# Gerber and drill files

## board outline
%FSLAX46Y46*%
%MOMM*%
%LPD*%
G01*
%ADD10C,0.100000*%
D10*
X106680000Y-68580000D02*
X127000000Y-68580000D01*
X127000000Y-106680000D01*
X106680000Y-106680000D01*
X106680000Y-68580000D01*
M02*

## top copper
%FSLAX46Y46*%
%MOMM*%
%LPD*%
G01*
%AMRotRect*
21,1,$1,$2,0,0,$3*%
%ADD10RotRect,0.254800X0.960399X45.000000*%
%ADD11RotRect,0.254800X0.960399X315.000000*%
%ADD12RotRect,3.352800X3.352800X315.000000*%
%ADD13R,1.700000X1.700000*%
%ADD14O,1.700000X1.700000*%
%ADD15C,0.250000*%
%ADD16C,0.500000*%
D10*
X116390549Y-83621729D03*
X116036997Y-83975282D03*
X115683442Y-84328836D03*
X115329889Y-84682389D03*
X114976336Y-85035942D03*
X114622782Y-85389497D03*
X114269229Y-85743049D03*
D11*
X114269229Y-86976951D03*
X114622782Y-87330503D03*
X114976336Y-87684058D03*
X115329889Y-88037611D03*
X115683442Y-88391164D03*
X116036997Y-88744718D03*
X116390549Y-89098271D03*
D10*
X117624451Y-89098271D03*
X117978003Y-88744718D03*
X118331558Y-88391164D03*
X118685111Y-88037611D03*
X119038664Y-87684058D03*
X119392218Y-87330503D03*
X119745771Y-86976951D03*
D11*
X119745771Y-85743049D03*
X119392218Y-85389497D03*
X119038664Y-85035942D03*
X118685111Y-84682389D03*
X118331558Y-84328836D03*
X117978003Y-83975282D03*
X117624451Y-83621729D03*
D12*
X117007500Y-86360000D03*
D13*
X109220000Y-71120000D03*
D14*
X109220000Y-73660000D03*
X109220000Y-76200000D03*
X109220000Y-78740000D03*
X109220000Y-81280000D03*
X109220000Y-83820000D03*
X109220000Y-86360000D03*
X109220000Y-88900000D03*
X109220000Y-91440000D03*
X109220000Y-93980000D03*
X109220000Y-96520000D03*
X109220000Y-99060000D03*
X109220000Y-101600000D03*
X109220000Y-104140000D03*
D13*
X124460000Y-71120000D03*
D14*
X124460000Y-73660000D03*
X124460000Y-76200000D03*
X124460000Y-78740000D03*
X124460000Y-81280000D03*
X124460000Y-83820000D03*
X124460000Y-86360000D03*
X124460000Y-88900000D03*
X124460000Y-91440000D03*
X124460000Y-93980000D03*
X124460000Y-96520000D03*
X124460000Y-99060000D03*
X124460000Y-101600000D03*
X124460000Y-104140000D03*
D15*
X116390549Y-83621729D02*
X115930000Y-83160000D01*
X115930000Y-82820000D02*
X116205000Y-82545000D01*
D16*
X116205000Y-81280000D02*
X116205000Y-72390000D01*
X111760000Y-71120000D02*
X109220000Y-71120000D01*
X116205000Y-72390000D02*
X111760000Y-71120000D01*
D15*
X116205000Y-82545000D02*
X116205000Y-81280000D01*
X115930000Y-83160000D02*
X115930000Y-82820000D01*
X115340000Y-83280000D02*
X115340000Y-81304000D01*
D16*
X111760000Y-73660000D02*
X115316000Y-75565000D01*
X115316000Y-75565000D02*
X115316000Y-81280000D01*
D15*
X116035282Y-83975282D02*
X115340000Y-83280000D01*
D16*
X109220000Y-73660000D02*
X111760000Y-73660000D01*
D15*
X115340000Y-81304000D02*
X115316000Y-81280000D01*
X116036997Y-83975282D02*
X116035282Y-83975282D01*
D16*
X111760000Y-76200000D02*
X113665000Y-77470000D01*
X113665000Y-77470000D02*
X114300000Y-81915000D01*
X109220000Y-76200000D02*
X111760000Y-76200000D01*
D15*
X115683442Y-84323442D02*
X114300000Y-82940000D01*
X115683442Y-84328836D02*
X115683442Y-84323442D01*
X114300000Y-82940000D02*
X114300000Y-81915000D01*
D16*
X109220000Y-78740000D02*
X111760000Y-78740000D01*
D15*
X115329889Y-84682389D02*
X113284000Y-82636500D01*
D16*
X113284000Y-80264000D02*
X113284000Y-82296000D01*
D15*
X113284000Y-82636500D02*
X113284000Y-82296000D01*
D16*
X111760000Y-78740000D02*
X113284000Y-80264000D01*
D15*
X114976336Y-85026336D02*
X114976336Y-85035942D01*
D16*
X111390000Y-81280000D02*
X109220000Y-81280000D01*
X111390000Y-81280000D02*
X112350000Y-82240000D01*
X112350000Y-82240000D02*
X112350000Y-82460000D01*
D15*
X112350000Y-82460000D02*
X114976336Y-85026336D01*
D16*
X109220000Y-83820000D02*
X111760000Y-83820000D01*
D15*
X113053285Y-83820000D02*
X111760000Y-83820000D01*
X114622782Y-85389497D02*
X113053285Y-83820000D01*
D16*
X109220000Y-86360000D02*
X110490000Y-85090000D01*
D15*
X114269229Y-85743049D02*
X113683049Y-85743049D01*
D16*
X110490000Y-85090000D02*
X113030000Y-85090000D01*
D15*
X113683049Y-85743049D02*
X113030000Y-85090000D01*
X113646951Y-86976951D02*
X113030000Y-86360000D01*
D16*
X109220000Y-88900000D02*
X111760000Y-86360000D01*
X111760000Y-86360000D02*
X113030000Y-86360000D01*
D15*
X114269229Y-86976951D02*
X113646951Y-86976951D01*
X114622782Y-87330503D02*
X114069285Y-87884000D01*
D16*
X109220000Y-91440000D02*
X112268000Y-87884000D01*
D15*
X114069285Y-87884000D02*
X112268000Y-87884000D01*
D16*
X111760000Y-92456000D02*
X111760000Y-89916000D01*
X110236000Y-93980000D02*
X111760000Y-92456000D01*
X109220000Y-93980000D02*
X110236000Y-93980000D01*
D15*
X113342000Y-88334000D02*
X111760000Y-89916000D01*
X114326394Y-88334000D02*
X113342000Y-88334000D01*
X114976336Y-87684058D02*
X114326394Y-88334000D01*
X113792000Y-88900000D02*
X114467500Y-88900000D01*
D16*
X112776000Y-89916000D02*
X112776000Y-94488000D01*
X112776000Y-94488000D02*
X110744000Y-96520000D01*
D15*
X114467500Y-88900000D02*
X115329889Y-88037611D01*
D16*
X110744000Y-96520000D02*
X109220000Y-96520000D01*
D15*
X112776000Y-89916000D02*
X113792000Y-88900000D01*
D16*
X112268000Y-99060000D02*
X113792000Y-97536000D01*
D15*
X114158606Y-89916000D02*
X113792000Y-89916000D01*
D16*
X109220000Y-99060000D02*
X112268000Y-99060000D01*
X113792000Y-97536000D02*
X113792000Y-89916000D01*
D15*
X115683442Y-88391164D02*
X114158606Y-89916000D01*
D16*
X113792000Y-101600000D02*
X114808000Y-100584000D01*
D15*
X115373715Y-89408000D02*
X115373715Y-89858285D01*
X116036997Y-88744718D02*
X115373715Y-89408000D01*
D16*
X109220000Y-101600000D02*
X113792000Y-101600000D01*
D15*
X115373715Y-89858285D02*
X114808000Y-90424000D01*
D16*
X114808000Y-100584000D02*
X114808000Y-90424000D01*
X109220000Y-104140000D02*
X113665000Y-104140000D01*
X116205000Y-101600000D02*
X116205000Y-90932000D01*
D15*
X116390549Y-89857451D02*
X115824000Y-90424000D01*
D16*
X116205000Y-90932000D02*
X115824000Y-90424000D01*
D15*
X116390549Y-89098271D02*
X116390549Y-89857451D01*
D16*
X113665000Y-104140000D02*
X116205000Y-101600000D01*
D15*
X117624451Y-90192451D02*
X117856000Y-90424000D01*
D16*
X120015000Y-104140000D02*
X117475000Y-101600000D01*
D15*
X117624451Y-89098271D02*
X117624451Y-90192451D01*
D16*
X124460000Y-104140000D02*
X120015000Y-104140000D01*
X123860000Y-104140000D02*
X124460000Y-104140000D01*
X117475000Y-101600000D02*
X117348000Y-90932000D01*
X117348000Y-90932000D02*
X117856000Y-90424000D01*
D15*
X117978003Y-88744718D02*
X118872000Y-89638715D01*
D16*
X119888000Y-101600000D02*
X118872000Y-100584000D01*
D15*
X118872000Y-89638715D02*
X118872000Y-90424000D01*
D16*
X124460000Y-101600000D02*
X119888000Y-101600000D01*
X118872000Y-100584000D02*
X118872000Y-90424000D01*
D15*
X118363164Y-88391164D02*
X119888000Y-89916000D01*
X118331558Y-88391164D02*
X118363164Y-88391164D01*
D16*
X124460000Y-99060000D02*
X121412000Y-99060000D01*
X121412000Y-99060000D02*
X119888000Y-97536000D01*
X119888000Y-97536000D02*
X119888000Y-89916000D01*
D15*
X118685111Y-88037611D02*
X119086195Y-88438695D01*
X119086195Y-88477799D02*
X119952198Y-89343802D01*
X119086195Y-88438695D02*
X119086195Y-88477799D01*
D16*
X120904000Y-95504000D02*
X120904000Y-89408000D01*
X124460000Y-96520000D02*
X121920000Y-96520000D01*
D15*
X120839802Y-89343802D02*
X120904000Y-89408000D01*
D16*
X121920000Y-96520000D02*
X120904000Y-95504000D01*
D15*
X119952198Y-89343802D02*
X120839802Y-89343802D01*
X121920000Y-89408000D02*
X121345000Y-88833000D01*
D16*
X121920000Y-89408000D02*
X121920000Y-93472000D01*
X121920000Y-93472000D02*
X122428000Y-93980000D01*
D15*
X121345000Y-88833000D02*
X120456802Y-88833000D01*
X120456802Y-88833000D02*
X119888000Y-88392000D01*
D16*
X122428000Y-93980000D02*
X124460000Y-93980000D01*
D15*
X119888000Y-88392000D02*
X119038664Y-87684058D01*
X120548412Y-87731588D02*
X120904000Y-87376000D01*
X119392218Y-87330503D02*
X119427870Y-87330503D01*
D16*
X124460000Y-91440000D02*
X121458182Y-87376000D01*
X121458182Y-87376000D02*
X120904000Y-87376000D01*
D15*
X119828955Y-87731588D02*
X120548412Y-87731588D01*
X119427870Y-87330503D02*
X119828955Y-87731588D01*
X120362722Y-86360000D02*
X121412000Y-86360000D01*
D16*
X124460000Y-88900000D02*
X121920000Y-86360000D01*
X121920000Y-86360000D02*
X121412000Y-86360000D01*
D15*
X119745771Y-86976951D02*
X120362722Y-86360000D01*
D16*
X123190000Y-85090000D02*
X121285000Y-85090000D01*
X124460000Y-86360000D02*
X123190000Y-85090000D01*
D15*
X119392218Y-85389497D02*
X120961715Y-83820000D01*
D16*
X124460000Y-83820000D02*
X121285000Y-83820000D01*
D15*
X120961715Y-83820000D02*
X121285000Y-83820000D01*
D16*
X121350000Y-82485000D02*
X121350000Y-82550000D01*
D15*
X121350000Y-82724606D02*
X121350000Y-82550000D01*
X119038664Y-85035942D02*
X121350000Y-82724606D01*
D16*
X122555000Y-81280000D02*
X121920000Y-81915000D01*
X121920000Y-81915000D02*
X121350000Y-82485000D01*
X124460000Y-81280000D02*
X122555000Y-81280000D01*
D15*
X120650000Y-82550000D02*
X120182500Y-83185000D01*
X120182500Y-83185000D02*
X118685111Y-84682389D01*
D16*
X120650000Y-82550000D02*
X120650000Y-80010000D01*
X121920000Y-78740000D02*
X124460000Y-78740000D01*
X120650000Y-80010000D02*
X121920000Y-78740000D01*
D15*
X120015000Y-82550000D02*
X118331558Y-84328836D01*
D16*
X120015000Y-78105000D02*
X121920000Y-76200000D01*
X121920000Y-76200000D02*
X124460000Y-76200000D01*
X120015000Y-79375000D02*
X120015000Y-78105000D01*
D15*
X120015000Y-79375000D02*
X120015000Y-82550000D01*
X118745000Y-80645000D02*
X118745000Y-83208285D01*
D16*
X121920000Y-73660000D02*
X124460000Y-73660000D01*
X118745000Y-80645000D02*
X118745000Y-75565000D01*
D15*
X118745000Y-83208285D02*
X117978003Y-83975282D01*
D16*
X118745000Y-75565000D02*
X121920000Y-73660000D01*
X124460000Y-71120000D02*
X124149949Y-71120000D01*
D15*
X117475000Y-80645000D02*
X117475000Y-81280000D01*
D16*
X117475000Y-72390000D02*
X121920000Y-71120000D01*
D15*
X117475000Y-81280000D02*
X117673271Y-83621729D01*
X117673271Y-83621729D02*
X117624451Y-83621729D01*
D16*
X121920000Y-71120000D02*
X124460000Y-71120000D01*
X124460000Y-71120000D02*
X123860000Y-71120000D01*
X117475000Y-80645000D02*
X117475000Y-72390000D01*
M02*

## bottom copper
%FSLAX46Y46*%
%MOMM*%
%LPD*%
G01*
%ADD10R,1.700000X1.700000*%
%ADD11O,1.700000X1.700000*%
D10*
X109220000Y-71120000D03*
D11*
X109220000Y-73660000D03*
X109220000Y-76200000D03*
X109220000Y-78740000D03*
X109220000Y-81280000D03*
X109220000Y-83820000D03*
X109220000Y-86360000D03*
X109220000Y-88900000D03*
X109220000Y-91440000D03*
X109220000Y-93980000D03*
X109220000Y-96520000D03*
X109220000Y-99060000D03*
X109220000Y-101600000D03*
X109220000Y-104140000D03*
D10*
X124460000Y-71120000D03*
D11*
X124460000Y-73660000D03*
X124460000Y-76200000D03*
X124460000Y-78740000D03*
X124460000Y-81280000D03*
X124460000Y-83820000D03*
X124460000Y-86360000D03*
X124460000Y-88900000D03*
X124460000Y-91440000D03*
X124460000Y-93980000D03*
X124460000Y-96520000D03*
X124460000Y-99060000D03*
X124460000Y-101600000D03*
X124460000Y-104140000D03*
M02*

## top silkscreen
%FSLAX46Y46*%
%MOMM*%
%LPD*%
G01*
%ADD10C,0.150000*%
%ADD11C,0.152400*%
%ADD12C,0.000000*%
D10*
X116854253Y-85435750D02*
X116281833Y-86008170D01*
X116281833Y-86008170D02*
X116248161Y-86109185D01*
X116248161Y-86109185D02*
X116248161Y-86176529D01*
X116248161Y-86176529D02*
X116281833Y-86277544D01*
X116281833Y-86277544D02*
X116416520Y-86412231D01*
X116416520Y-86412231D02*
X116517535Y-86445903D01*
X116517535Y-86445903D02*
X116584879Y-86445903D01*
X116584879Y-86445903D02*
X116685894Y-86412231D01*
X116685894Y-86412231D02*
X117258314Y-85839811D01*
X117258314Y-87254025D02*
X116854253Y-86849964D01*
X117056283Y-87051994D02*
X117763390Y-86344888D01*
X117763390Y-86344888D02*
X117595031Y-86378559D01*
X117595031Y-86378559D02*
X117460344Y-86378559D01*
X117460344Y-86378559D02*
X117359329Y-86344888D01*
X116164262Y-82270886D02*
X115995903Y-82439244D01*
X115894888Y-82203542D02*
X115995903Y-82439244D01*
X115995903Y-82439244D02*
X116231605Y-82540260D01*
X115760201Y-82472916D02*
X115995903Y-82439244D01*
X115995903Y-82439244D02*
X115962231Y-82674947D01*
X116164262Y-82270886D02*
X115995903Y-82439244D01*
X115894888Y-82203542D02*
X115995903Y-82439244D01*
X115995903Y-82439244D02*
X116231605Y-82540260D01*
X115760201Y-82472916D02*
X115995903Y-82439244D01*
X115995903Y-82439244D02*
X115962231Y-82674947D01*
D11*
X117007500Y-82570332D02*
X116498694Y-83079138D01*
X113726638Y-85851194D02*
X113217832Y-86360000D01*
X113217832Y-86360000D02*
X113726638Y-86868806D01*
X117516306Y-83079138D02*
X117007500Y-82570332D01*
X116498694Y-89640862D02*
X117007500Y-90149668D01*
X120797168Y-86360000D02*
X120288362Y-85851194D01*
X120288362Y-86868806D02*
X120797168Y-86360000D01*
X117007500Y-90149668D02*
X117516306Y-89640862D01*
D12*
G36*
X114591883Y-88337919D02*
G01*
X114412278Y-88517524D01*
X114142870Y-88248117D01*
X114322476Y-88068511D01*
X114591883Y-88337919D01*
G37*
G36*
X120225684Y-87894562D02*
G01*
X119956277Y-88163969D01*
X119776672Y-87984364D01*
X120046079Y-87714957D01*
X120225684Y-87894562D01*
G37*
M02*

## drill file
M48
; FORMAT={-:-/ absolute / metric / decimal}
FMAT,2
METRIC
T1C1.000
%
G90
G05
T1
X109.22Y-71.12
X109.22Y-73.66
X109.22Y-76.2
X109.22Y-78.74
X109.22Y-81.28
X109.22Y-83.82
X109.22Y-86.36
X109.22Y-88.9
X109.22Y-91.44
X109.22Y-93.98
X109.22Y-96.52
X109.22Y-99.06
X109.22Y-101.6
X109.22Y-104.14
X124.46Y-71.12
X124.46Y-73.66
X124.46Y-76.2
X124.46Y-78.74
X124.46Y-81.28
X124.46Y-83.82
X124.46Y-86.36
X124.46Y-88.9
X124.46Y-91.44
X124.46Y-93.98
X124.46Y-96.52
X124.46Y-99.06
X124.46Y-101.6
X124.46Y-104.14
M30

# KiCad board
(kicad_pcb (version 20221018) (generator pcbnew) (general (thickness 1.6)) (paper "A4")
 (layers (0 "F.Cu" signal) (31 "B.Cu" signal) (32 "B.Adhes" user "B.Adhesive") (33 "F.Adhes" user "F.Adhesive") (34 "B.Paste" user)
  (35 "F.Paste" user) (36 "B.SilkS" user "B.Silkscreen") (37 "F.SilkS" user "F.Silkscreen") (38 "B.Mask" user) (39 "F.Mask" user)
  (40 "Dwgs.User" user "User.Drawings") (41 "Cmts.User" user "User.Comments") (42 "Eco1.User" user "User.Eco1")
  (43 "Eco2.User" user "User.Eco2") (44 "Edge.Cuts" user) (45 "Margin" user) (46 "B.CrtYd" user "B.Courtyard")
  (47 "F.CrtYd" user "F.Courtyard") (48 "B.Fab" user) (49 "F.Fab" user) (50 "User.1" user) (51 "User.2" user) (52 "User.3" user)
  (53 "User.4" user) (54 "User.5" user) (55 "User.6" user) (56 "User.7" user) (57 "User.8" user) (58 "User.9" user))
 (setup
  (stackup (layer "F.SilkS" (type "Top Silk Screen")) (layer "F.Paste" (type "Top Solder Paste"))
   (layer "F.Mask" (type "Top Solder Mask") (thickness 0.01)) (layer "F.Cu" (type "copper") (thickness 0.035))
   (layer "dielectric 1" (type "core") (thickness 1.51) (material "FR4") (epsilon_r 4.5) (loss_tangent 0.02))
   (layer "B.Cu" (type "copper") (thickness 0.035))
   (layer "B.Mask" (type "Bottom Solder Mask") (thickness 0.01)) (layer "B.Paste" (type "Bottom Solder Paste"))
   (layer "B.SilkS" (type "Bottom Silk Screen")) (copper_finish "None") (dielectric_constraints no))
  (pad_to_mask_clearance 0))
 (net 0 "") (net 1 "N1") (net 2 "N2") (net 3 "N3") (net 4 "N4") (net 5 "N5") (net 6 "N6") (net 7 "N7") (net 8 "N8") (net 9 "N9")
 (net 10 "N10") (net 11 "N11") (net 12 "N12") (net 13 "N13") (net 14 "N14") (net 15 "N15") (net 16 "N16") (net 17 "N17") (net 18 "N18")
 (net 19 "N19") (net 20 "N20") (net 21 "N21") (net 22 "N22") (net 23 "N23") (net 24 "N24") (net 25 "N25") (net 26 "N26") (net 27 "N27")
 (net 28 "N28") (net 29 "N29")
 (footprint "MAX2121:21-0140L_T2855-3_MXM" (layer "F.Cu") (at 117.0075 86.36 -45)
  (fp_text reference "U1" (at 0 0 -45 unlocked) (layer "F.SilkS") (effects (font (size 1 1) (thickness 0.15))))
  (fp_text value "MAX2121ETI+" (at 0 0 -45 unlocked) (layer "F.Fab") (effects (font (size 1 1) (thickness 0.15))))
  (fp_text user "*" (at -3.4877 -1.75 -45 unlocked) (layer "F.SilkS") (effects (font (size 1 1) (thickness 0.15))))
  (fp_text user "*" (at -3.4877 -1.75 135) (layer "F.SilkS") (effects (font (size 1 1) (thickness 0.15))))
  (fp_line (start -2.6797 -2.6797) (end -2.6797 -1.96014) (stroke (width 0.1524) (type solid)) (layer "F.SilkS"))
  (fp_line (start -2.6797 1.96014) (end -2.6797 2.6797) (stroke (width 0.1524) (type solid)) (layer "F.SilkS"))
  (fp_line (start -2.6797 2.6797) (end -1.96014 2.6797) (stroke (width 0.1524) (type solid)) (layer "F.SilkS"))
  (fp_line (start -1.96014 -2.6797) (end -2.6797 -2.6797) (stroke (width 0.1524) (type solid)) (layer "F.SilkS"))
  (fp_line (start 1.96014 2.6797) (end 2.6797 2.6797) (stroke (width 0.1524) (type solid)) (layer "F.SilkS"))
  (fp_line (start 2.6797 -2.6797) (end 1.96014 -2.6797) (stroke (width 0.1524) (type solid)) (layer "F.SilkS"))
  (fp_line (start 2.6797 -1.96014) (end 2.6797 -2.6797) (stroke (width 0.1524) (type solid)) (layer "F.SilkS"))
  (fp_line (start 2.6797 2.6797) (end 2.6797 1.96014) (stroke (width 0.1524) (type solid)) (layer "F.SilkS"))
  (fp_poly
   (pts (xy -0.690499 3.106699) (xy -0.690499 3.360699) (xy -0.309499 3.360699) (xy -0.309499 3.106699)) (stroke (width 0) (type solid))
   (fill solid) (layer "F.SilkS"))
  (fp_poly
   (pts (xy 3.360699 -1.190501) (xy 3.360699 -0.809501) (xy 3.106699 -0.809501) (xy 3.106699 -1.190501)) (stroke (width 0) (type solid))
   (fill solid) (layer "F.SilkS"))
  (pad "1" smd rect (at -2.3725 -1.5 45) (size 0.2548 0.960399) (layers "F.Cu" "F.Paste" "F.Mask") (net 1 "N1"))
  (pad "2" smd rect (at -2.3725 -1.000001 45) (size 0.2548 0.960399) (layers "F.Cu" "F.Paste" "F.Mask") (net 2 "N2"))
  (pad "3" smd rect (at -2.3725 -0.499999 45) (size 0.2548 0.960399) (layers "F.Cu" "F.Paste" "F.Mask") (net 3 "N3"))
  (pad "4" smd rect (at -2.3725 0 45) (size 0.2548 0.960399) (layers "F.Cu" "F.Paste" "F.Mask") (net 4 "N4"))
  (pad "5" smd rect (at -2.3725 0.499999 45) (size 0.2548 0.960399) (layers "F.Cu" "F.Paste" "F.Mask") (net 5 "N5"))
  (pad "6" smd rect (at -2.3725 1.000001 45) (size 0.2548 0.960399) (layers "F.Cu" "F.Paste" "F.Mask") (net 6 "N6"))
  (pad "7" smd rect (at -2.3725 1.5 45) (size 0.2548 0.960399) (layers "F.Cu" "F.Paste" "F.Mask") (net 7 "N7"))
  (pad "8" smd rect (at -1.5 2.3725 315) (size 0.2548 0.960399) (layers "F.Cu" "F.Paste" "F.Mask") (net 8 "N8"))
  (pad "9" smd rect (at -1.000001 2.3725 315) (size 0.2548 0.960399) (layers "F.Cu" "F.Paste" "F.Mask") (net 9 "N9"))
  (pad "10" smd rect (at -0.499999 2.3725 315) (size 0.2548 0.960399) (layers "F.Cu" "F.Paste" "F.Mask") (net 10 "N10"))
  (pad "11" smd rect (at 0 2.3725 315) (size 0.2548 0.960399) (layers "F.Cu" "F.Paste" "F.Mask") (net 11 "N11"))
  (pad "12" smd rect (at 0.499999 2.3725 315) (size 0.2548 0.960399) (layers "F.Cu" "F.Paste" "F.Mask") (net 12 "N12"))
  (pad "13" smd rect (at 1.000001 2.3725 315) (size 0.2548 0.960399) (layers "F.Cu" "F.Paste" "F.Mask") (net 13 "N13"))
  (pad "14" smd rect (at 1.5 2.3725 315) (size 0.2548 0.960399) (layers "F.Cu" "F.Paste" "F.Mask") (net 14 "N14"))
  (pad "15" smd rect (at 2.3725 1.5 45) (size 0.2548 0.960399) (layers "F.Cu" "F.Paste" "F.Mask") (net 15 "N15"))
  (pad "16" smd rect (at 2.3725 1.000001 45) (size 0.2548 0.960399) (layers "F.Cu" "F.Paste" "F.Mask") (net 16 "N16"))
  (pad "17" smd rect (at 2.3725 0.499999 45) (size 0.2548 0.960399) (layers "F.Cu" "F.Paste" "F.Mask") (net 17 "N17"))
  (pad "18" smd rect (at 2.3725 0 45) (size 0.2548 0.960399) (layers "F.Cu" "F.Paste" "F.Mask") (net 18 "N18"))
  (pad "19" smd rect (at 2.3725 -0.499999 45) (size 0.2548 0.960399) (layers "F.Cu" "F.Paste" "F.Mask") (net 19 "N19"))
  (pad "20" smd rect (at 2.3725 -1.000001 45) (size 0.2548 0.960399) (layers "F.Cu" "F.Paste" "F.Mask") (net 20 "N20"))
  (pad "21" smd rect (at 2.3725 -1.5 45) (size 0.2548 0.960399) (layers "F.Cu" "F.Paste" "F.Mask") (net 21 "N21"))
  (pad "22" smd rect (at 1.5 -2.3725 315) (size 0.2548 0.960399) (layers "F.Cu" "F.Paste" "F.Mask") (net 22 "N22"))
  (pad "23" smd rect (at 1.000001 -2.3725 315) (size 0.2548 0.960399) (layers "F.Cu" "F.Paste" "F.Mask") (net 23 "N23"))
  (pad "24" smd rect (at 0.499999 -2.3725 315) (size 0.2548 0.960399) (layers "F.Cu" "F.Paste" "F.Mask") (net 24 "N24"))
  (pad "25" smd rect (at 0 -2.3725 315) (size 0.2548 0.960399) (layers "F.Cu" "F.Paste" "F.Mask") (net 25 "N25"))
  (pad "26" smd rect (at -0.499999 -2.3725 315) (size 0.2548 0.960399) (layers "F.Cu" "F.Paste" "F.Mask") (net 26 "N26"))
  (pad "27" smd rect (at -1.000001 -2.3725 315) (size 0.2548 0.960399) (layers "F.Cu" "F.Paste" "F.Mask") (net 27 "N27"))
  (pad "28" smd rect (at -1.5 -2.3725 315) (size 0.2548 0.960399) (layers "F.Cu" "F.Paste" "F.Mask") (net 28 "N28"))
  (pad "29" smd rect (at 0 0 315) (size 3.3528 3.3528) (layers "F.Cu" "F.Mask") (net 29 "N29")))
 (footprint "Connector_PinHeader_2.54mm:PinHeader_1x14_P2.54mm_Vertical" (layer "B.Cu") (at 109.22 71.12 180)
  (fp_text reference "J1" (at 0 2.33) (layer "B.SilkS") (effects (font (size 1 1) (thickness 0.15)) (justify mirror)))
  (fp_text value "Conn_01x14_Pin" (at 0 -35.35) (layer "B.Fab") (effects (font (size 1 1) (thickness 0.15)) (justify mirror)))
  (pad "1" thru_hole rect (at 0 0 180) (size 1.7 1.7) (drill 1) (layers "*.Cu" "*.Mask") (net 1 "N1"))
  (pad "2" thru_hole oval (at 0 -2.54 180) (size 1.7 1.7) (drill 1) (layers "*.Cu" "*.Mask") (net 2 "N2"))
  (pad "3" thru_hole oval (at 0 -5.08 180) (size 1.7 1.7) (drill 1) (layers "*.Cu" "*.Mask") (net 3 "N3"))
  (pad "4" thru_hole oval (at 0 -7.62 180) (size 1.7 1.7) (drill 1) (layers "*.Cu" "*.Mask") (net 4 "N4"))
  (pad "5" thru_hole oval (at 0 -10.16 180) (size 1.7 1.7) (drill 1) (layers "*.Cu" "*.Mask") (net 5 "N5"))
  (pad "6" thru_hole oval (at 0 -12.7 180) (size 1.7 1.7) (drill 1) (layers "*.Cu" "*.Mask") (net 6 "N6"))
  (pad "7" thru_hole oval (at 0 -15.24 180) (size 1.7 1.7) (drill 1) (layers "*.Cu" "*.Mask") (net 7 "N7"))
  (pad "8" thru_hole oval (at 0 -17.78 180) (size 1.7 1.7) (drill 1) (layers "*.Cu" "*.Mask") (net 8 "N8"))
  (pad "9" thru_hole oval (at 0 -20.32 180) (size 1.7 1.7) (drill 1) (layers "*.Cu" "*.Mask") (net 9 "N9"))
  (pad "10" thru_hole oval (at 0 -22.86 180) (size 1.7 1.7) (drill 1) (layers "*.Cu" "*.Mask") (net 10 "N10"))
  (pad "11" thru_hole oval (at 0 -25.4 180) (size 1.7 1.7) (drill 1) (layers "*.Cu" "*.Mask") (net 11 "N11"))
  (pad "12" thru_hole oval (at 0 -27.94 180) (size 1.7 1.7) (drill 1) (layers "*.Cu" "*.Mask") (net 12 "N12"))
  (pad "13" thru_hole oval (at 0 -30.48 180) (size 1.7 1.7) (drill 1) (layers "*.Cu" "*.Mask") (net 13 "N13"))
  (pad "14" thru_hole oval (at 0 -33.02 180) (size 1.7 1.7) (drill 1) (layers "*.Cu" "*.Mask") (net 14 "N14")))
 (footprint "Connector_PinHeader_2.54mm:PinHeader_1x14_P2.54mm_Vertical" (layer "B.Cu") (at 124.46 71.12 180)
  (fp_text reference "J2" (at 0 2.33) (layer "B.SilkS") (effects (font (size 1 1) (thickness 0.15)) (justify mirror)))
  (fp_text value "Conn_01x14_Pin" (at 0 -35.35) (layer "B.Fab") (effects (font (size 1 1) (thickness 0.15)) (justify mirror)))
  (pad "1" thru_hole rect (at 0 0 180) (size 1.7 1.7) (drill 1) (layers "*.Cu" "*.Mask") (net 28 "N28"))
  (pad "2" thru_hole oval (at 0 -2.54 180) (size 1.7 1.7) (drill 1) (layers "*.Cu" "*.Mask") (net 27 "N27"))
  (pad "3" thru_hole oval (at 0 -5.08 180) (size 1.7 1.7) (drill 1) (layers "*.Cu" "*.Mask") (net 26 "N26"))
  (pad "4" thru_hole oval (at 0 -7.62 180) (size 1.7 1.7) (drill 1) (layers "*.Cu" "*.Mask") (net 25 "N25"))
  (pad "5" thru_hole oval (at 0 -10.16 180) (size 1.7 1.7) (drill 1) (layers "*.Cu" "*.Mask") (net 24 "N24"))
  (pad "6" thru_hole oval (at 0 -12.7 180) (size 1.7 1.7) (drill 1) (layers "*.Cu" "*.Mask") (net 23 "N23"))
  (pad "7" thru_hole oval (at 0 -15.24 180) (size 1.7 1.7) (drill 1) (layers "*.Cu" "*.Mask") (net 22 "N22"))
  (pad "8" thru_hole oval (at 0 -17.78 180) (size 1.7 1.7) (drill 1) (layers "*.Cu" "*.Mask") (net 21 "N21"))
  (pad "9" thru_hole oval (at 0 -20.32 180) (size 1.7 1.7) (drill 1) (layers "*.Cu" "*.Mask") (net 20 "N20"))
  (pad "10" thru_hole oval (at 0 -22.86 180) (size 1.7 1.7) (drill 1) (layers "*.Cu" "*.Mask") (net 19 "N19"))
  (pad "11" thru_hole oval (at 0 -25.4 180) (size 1.7 1.7) (drill 1) (layers "*.Cu" "*.Mask") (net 18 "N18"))
  (pad "12" thru_hole oval (at 0 -27.94 180) (size 1.7 1.7) (drill 1) (layers "*.Cu" "*.Mask") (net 17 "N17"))
  (pad "13" thru_hole oval (at 0 -30.48 180) (size 1.7 1.7) (drill 1) (layers "*.Cu" "*.Mask") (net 16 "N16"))
  (pad "14" thru_hole oval (at 0 -33.02 180) (size 1.7 1.7) (drill 1) (layers "*.Cu" "*.Mask") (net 15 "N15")))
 (gr_rect (start 106.68 68.58) (end 127 106.68) (stroke (width 0.1) (type default)) (fill none) (layer "Edge.Cuts"))
 (segment (start 116.390549 83.621729) (end 115.93 83.16) (width 0.25) (layer "F.Cu") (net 1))
 (segment (start 115.93 82.82) (end 116.205 82.545) (width 0.25) (layer "F.Cu") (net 1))
 (segment (start 116.205 81.28) (end 116.205 72.39) (width 0.5) (layer "F.Cu") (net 1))
 (segment (start 111.76 71.12) (end 109.22 71.12) (width 0.5) (layer "F.Cu") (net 1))
 (segment (start 116.205 72.39) (end 111.76 71.12) (width 0.5) (layer "F.Cu") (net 1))
 (segment (start 116.205 82.545) (end 116.205 81.28) (width 0.25) (layer "F.Cu") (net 1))
 (segment (start 115.93 83.16) (end 115.93 82.82) (width 0.25) (layer "F.Cu") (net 1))
 (segment (start 115.34 83.28) (end 115.34 81.304) (width 0.25) (layer "F.Cu") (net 2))
 (segment (start 111.76 73.66) (end 115.316 75.565) (width 0.5) (layer "F.Cu") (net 2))
 (segment (start 115.316 75.565) (end 115.316 81.28) (width 0.5) (layer "F.Cu") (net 2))
 (segment (start 116.035282 83.975282) (end 115.34 83.28) (width 0.25) (layer "F.Cu") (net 2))
 (segment (start 109.22 73.66) (end 111.76 73.66) (width 0.5) (layer "F.Cu") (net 2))
 (segment (start 115.34 81.304) (end 115.316 81.28) (width 0.25) (layer "F.Cu") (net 2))
 (segment (start 116.036997 83.975282) (end 116.035282 83.975282) (width 0.25) (layer "F.Cu") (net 2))
 (segment (start 111.76 76.2) (end 113.665 77.47) (width 0.5) (layer "F.Cu") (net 3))
 (segment (start 113.665 77.47) (end 114.3 81.915) (width 0.5) (layer "F.Cu") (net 3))
 (segment (start 109.22 76.2) (end 111.76 76.2) (width 0.5) (layer "F.Cu") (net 3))
 (segment (start 115.683442 84.323442) (end 114.3 82.94) (width 0.25) (layer "F.Cu") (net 3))
 (segment (start 115.683442 84.328836) (end 115.683442 84.323442) (width 0.25) (layer "F.Cu") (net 3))
 (segment (start 114.3 82.94) (end 114.3 81.915) (width 0.25) (layer "F.Cu") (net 3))
 (segment (start 109.22 78.74) (end 111.76 78.74) (width 0.5) (layer "F.Cu") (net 4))
 (segment (start 115.329889 84.682389) (end 113.284 82.6365) (width 0.25) (layer "F.Cu") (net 4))
 (segment (start 113.284 80.264) (end 113.284 82.296) (width 0.5) (layer "F.Cu") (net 4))
 (segment (start 113.284 82.6365) (end 113.284 82.296) (width 0.25) (layer "F.Cu") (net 4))
 (segment (start 111.76 78.74) (end 113.284 80.264) (width 0.5) (layer "F.Cu") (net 4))
 (segment (start 114.976336 85.026336) (end 114.976336 85.035942) (width 0.25) (layer "F.Cu") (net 5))
 (segment (start 111.39 81.28) (end 109.22 81.28) (width 0.5) (layer "F.Cu") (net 5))
 (segment (start 111.39 81.28) (end 112.35 82.24) (width 0.5) (layer "F.Cu") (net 5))
 (segment (start 112.35 82.24) (end 112.35 82.46) (width 0.5) (layer "F.Cu") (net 5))
 (segment (start 112.35 82.46) (end 114.976336 85.026336) (width 0.25) (layer "F.Cu") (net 5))
 (segment (start 109.22 83.82) (end 111.76 83.82) (width 0.5) (layer "F.Cu") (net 6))
 (segment (start 113.053285 83.82) (end 111.76 83.82) (width 0.25) (layer "F.Cu") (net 6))
 (segment (start 114.622782 85.389497) (end 113.053285 83.82) (width 0.25) (layer "F.Cu") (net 6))
 (segment (start 109.22 86.36) (end 110.49 85.09) (width 0.5) (layer "F.Cu") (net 7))
 (segment (start 114.269229 85.743049) (end 113.683049 85.743049) (width 0.25) (layer "F.Cu") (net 7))
 (segment (start 110.49 85.09) (end 113.03 85.09) (width 0.5) (layer "F.Cu") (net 7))
 (segment (start 113.683049 85.743049) (end 113.03 85.09) (width 0.25) (layer "F.Cu") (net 7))
 (segment (start 113.646951 86.976951) (end 113.03 86.36) (width 0.25) (layer "F.Cu") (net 8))
 (segment (start 109.22 88.9) (end 111.76 86.36) (width 0.5) (layer "F.Cu") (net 8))
 (segment (start 111.76 86.36) (end 113.03 86.36) (width 0.5) (layer "F.Cu") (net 8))
 (segment (start 114.269229 86.976951) (end 113.646951 86.976951) (width 0.25) (layer "F.Cu") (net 8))
 (segment (start 114.622782 87.330503) (end 114.069285 87.884) (width 0.25) (layer "F.Cu") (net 9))
 (segment (start 109.22 91.44) (end 112.268 87.884) (width 0.5) (layer "F.Cu") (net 9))
 (segment (start 114.069285 87.884) (end 112.268 87.884) (width 0.25) (layer "F.Cu") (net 9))
 (segment (start 111.76 92.456) (end 111.76 89.916) (width 0.5) (layer "F.Cu") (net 10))
 (segment (start 110.236 93.98) (end 111.76 92.456) (width 0.5) (layer "F.Cu") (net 10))
 (segment (start 109.22 93.98) (end 110.236 93.98) (width 0.5) (layer "F.Cu") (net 10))
 (segment (start 113.342 88.334) (end 111.76 89.916) (width 0.25) (layer "F.Cu") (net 10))
 (segment (start 114.326394 88.334) (end 113.342 88.334) (width 0.25) (layer "F.Cu") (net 10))
 (segment (start 114.976336 87.684058) (end 114.326394 88.334) (width 0.25) (layer "F.Cu") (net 10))
 (segment (start 113.792 88.9) (end 114.4675 88.9) (width 0.25) (layer "F.Cu") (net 11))
 (segment (start 112.776 89.916) (end 112.776 94.488) (width 0.5) (layer "F.Cu") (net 11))
 (segment (start 112.776 94.488) (end 110.744 96.52) (width 0.5) (layer "F.Cu") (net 11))
 (segment (start 114.4675 88.9) (end 115.329889 88.037611) (width 0.25) (layer "F.Cu") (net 11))
 (segment (start 110.744 96.52) (end 109.22 96.52) (width 0.5) (layer "F.Cu") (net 11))
 (segment (start 112.776 89.916) (end 113.792 88.9) (width 0.25) (layer "F.Cu") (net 11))
 (segment (start 112.268 99.06) (end 113.792 97.536) (width 0.5) (layer "F.Cu") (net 12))
 (segment (start 114.158606 89.916) (end 113.792 89.916) (width 0.25) (layer "F.Cu") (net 12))
 (segment (start 109.22 99.06) (end 112.268 99.06) (width 0.5) (layer "F.Cu") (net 12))
 (segment (start 113.792 97.536) (end 113.792 89.916) (width 0.5) (layer "F.Cu") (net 12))
 (segment (start 115.683442 88.391164) (end 114.158606 89.916) (width 0.25) (layer "F.Cu") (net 12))
 (segment (start 113.792 101.6) (end 114.808 100.584) (width 0.5) (layer "F.Cu") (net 13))
 (segment (start 115.373715 89.408) (end 115.373715 89.858285) (width 0.25) (layer "F.Cu") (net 13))
 (segment (start 116.036997 88.744718) (end 115.373715 89.408) (width 0.25) (layer "F.Cu") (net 13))
 (segment (start 109.22 101.6) (end 113.792 101.6) (width 0.5) (layer "F.Cu") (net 13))
 (segment (start 115.373715 89.858285) (end 114.808 90.424) (width 0.25) (layer "F.Cu") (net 13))
 (segment (start 114.808 100.584) (end 114.808 90.424) (width 0.5) (layer "F.Cu") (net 13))
 (segment (start 109.22 104.14) (end 113.665 104.14) (width 0.5) (layer "F.Cu") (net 14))
 (segment (start 116.205 101.6) (end 116.205 90.932) (width 0.5) (layer "F.Cu") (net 14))
 (segment (start 116.390549 89.857451) (end 115.824 90.424) (width 0.25) (layer "F.Cu") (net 14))
 (segment (start 116.205 90.932) (end 115.824 90.424) (width 0.5) (layer "F.Cu") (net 14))
 (segment (start 116.390549 89.098271) (end 116.390549 89.857451) (width 0.25) (layer "F.Cu") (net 14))
 (segment (start 113.665 104.14) (end 116.205 101.6) (width 0.5) (layer "F.Cu") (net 14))
 (segment (start 117.624451 90.192451) (end 117.856 90.424) (width 0.25) (layer "F.Cu") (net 15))
 (segment (start 120.015 104.14) (end 117.475 101.6) (width 0.5) (layer "F.Cu") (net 15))
 (segment (start 117.624451 89.098271) (end 117.624451 90.192451) (width 0.25) (layer "F.Cu") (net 15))
 (segment (start 124.46 104.14) (end 120.015 104.14) (width 0.5) (layer "F.Cu") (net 15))
 (segment (start 123.86 104.14) (end 124.46 104.14) (width 0.5) (layer "F.Cu") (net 15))
 (segment (start 117.475 101.6) (end 117.348 90.932) (width 0.5) (layer "F.Cu") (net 15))
 (segment (start 117.348 90.932) (end 117.856 90.424) (width 0.5) (layer "F.Cu") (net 15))
 (segment (start 117.978003 88.744718) (end 118.872 89.638715) (width 0.25) (layer "F.Cu") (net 16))
 (segment (start 119.888 101.6) (end 118.872 100.584) (width 0.5) (layer "F.Cu") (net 16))
 (segment (start 118.872 89.638715) (end 118.872 90.424) (width 0.25) (layer "F.Cu") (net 16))
 (segment (start 124.46 101.6) (end 119.888 101.6) (width 0.5) (layer "F.Cu") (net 16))
 (segment (start 118.872 100.584) (end 118.872 90.424) (width 0.5) (layer "F.Cu") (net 16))
 (segment (start 118.363164 88.391164) (end 119.888 89.916) (width 0.25) (layer "F.Cu") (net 17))
 (segment (start 118.331558 88.391164) (end 118.363164 88.391164) (width 0.25) (layer "F.Cu") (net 17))
 (segment (start 124.46 99.06) (end 121.412 99.06) (width 0.5) (layer "F.Cu") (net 17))
 (segment (start 121.412 99.06) (end 119.888 97.536) (width 0.5) (layer "F.Cu") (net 17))
 (segment (start 119.888 97.536) (end 119.888 89.916) (width 0.5) (layer "F.Cu") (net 17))
 (segment (start 118.685111 88.037611) (end 119.086195 88.438695) (width 0.25) (layer "F.Cu") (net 18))
 (segment (start 119.086195 88.477799) (end 119.952198 89.343802) (width 0.25) (layer "F.Cu") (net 18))
 (segment (start 119.086195 88.438695) (end 119.086195 88.477799) (width 0.25) (layer "F.Cu") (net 18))
 (segment (start 120.904 95.504) (end 120.904 89.408) (width 0.5) (layer "F.Cu") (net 18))
 (segment (start 124.46 96.52) (end 121.92 96.52) (width 0.5) (layer "F.Cu") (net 18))
 (segment (start 120.839802 89.343802) (end 120.904 89.408) (width 0.25) (layer "F.Cu") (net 18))
 (segment (start 121.92 96.52) (end 120.904 95.504) (width 0.5) (layer "F.Cu") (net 18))
 (segment (start 119.952198 89.343802) (end 120.839802 89.343802) (width 0.25) (layer "F.Cu") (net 18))
 (segment (start 121.92 89.408) (end 121.345 88.833) (width 0.25) (layer "F.Cu") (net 19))
 (segment (start 121.92 89.408) (end 121.92 93.472) (width 0.5) (layer "F.Cu") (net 19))
 (segment (start 121.92 93.472) (end 122.428 93.98) (width 0.5) (layer "F.Cu") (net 19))
 (segment (start 121.345 88.833) (end 120.456802 88.833) (width 0.25) (layer "F.Cu") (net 19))
 (segment (start 120.456802 88.833) (end 119.888 88.392) (width 0.25) (layer "F.Cu") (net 19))
 (segment (start 122.428 93.98) (end 124.46 93.98) (width 0.5) (layer "F.Cu") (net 19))
 (segment (start 119.888 88.392) (end 119.038664 87.684058) (width 0.25) (layer "F.Cu") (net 19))
 (segment (start 120.548412 87.731588) (end 120.904 87.376) (width 0.25) (layer "F.Cu") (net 20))
 (segment (start 119.392218 87.330503) (end 119.42787 87.330503) (width 0.25) (layer "F.Cu") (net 20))
 (segment (start 124.46 91.44) (end 121.458182 87.376) (width 0.5) (layer "F.Cu") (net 20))
 (segment (start 121.458182 87.376) (end 120.904 87.376) (width 0.5) (layer "F.Cu") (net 20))
 (segment (start 119.828955 87.731588) (end 120.548412 87.731588) (width 0.25) (layer "F.Cu") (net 20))
 (segment (start 119.42787 87.330503) (end 119.828955 87.731588) (width 0.25) (layer "F.Cu") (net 20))
 (segment (start 120.362722 86.36) (end 121.412 86.36) (width 0.25) (layer "F.Cu") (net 21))
 (segment (start 124.46 88.9) (end 121.92 86.36) (width 0.5) (layer "F.Cu") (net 21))
 (segment (start 121.92 86.36) (end 121.412 86.36) (width 0.5) (layer "F.Cu") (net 21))
 (segment (start 119.745771 86.976951) (end 120.362722 86.36) (width 0.25) (layer "F.Cu") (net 21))
 (segment (start 123.19 85.09) (end 121.285 85.09) (width 0.5) (layer "F.Cu") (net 22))
 (segment (start 124.46 86.36) (end 123.19 85.09) (width 0.5) (layer "F.Cu") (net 22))
 (segment (start 119.392218 85.389497) (end 120.961715 83.82) (width 0.25) (layer "F.Cu") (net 23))
 (segment (start 124.46 83.82) (end 121.285 83.82) (width 0.5) (layer "F.Cu") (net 23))
 (segment (start 120.961715 83.82) (end 121.285 83.82) (width 0.25) (layer "F.Cu") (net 23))
 (segment (start 121.35 82.485) (end 121.35 82.55) (width 0.5) (layer "F.Cu") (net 24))
 (segment (start 121.35 82.724606) (end 121.35 82.55) (width 0.25) (layer "F.Cu") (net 24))
 (segment (start 119.038664 85.035942) (end 121.35 82.724606) (width 0.25) (layer "F.Cu") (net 24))
 (segment (start 122.555 81.28) (end 121.92 81.915) (width 0.5) (layer "F.Cu") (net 24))
 (segment (start 121.92 81.915) (end 121.35 82.485) (width 0.5) (layer "F.Cu") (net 24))
 (segment (start 124.46 81.28) (end 122.555 81.28) (width 0.5) (layer "F.Cu") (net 24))
 (segment (start 120.65 82.55) (end 120.1825 83.185) (width 0.25) (layer "F.Cu") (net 25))
 (segment (start 120.1825 83.185) (end 118.685111 84.682389) (width 0.25) (layer "F.Cu") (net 25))
 (segment (start 120.65 82.55) (end 120.65 80.01) (width 0.5) (layer "F.Cu") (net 25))
 (segment (start 121.92 78.74) (end 124.46 78.74) (width 0.5) (layer "F.Cu") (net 25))
 (segment (start 120.65 80.01) (end 121.92 78.74) (width 0.5) (layer "F.Cu") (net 25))
 (segment (start 120.015 82.55) (end 118.331558 84.328836) (width 0.25) (layer "F.Cu") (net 26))
 (segment (start 120.015 78.105) (end 121.92 76.2) (width 0.5) (layer "F.Cu") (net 26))
 (segment (start 121.92 76.2) (end 124.46 76.2) (width 0.5) (layer "F.Cu") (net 26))
 (segment (start 120.015 79.375) (end 120.015 78.105) (width 0.5) (layer "F.Cu") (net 26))
 (segment (start 120.015 79.375) (end 120.015 82.55) (width 0.25) (layer "F.Cu") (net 26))
 (segment (start 118.745 80.645) (end 118.745 83.208285) (width 0.25) (layer "F.Cu") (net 27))
 (segment (start 121.92 73.66) (end 124.46 73.66) (width 0.5) (layer "F.Cu") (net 27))
 (segment (start 118.745 80.645) (end 118.745 75.565) (width 0.5) (layer "F.Cu") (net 27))
 (segment (start 118.745 83.208285) (end 117.978003 83.975282) (width 0.25) (layer "F.Cu") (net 27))
 (segment (start 118.745 75.565) (end 121.92 73.66) (width 0.5) (layer "F.Cu") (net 27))
 (segment (start 124.46 71.12) (end 124.149949 71.12) (width 0.5) (layer "F.Cu") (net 28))
 (segment (start 117.475 80.645) (end 117.475 81.28) (width 0.25) (layer "F.Cu") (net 28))
 (segment (start 117.475 72.39) (end 121.92 71.12) (width 0.5) (layer "F.Cu") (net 28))
 (segment (start 117.475 81.28) (end 117.673271 83.621729) (width 0.25) (layer "F.Cu") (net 28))
 (segment (start 117.673271 83.621729) (end 117.624451 83.621729) (width 0.25) (layer "F.Cu") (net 28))
 (segment (start 121.92 71.12) (end 124.46 71.12) (width 0.5) (layer "F.Cu") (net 28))
 (segment (start 124.46 71.12) (end 123.86 71.12) (width 0.5) (layer "F.Cu") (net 28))
 (segment (start 117.475 80.645) (end 117.475 72.39) (width 0.5) (layer "F.Cu") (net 28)))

